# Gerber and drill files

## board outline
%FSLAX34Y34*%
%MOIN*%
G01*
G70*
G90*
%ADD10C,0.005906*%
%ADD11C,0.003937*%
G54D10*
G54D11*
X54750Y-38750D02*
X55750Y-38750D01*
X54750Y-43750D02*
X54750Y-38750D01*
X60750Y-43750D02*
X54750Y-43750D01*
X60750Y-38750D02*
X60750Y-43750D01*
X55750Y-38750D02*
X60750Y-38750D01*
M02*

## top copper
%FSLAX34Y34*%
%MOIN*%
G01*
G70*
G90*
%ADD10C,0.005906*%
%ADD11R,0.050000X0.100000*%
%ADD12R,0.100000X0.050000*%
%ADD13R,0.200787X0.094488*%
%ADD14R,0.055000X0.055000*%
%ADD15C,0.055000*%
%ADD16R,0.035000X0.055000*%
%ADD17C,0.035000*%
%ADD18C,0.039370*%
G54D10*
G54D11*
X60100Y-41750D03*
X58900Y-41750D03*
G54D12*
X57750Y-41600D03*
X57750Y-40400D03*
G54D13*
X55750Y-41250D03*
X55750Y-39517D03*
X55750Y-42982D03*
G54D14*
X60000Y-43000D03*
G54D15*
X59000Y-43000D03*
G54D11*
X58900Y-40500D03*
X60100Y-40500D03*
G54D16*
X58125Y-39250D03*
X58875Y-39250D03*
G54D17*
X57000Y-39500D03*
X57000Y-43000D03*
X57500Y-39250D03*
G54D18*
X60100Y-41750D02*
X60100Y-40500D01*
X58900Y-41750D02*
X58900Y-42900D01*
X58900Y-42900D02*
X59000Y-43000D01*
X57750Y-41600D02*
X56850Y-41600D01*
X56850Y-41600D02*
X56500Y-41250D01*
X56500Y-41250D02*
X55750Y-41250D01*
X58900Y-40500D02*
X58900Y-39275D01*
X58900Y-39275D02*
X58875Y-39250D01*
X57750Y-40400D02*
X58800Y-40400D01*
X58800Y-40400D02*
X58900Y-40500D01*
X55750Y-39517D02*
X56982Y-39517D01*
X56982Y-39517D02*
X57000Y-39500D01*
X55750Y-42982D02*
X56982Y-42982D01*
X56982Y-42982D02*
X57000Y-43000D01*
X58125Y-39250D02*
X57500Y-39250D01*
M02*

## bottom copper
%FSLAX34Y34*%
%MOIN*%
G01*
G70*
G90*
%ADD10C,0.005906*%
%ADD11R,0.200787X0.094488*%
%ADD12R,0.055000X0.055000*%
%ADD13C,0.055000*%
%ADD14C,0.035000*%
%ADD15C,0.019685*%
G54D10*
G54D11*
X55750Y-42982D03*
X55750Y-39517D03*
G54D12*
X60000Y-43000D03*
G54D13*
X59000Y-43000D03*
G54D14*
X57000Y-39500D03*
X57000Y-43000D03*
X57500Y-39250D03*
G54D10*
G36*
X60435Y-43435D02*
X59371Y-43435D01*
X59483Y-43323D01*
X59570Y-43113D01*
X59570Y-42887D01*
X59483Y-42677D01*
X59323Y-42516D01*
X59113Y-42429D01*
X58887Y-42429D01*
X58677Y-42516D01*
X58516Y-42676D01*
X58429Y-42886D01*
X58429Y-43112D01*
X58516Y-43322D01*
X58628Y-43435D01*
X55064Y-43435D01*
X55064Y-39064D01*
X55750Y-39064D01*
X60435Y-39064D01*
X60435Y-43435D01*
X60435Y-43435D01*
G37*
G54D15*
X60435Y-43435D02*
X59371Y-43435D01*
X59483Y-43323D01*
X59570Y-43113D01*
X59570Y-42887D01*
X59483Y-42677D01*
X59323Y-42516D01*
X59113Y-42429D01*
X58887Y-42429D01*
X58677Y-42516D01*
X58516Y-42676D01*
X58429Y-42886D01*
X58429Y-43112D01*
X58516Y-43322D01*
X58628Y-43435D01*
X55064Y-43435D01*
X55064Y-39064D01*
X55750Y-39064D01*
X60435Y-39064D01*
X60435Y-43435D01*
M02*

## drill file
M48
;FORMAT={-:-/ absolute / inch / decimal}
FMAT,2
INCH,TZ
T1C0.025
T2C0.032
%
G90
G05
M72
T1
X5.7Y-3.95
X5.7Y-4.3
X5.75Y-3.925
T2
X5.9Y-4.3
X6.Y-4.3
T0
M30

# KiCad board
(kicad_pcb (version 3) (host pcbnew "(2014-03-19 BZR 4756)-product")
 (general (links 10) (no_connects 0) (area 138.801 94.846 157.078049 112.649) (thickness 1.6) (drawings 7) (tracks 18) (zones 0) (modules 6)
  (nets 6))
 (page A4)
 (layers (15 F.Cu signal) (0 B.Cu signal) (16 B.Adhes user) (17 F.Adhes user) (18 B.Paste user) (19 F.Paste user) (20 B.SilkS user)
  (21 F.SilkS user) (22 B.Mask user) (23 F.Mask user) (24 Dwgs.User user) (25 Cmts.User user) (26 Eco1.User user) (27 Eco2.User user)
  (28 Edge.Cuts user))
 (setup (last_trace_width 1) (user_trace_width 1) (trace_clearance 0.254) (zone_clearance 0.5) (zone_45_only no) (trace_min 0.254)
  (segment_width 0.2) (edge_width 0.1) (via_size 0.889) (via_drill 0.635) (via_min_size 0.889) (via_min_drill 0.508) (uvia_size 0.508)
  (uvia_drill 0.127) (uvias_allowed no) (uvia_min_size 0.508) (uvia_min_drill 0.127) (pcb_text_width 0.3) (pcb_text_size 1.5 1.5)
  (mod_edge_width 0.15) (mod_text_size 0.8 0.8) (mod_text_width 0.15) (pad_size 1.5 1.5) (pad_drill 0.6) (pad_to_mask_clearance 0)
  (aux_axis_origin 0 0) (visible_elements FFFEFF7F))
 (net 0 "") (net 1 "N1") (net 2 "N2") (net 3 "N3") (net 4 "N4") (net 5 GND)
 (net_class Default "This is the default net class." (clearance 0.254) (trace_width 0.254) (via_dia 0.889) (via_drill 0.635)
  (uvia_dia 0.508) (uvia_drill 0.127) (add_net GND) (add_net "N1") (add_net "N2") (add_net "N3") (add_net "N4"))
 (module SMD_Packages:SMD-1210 (layer F.Cu) (at 151.13 106.045 180)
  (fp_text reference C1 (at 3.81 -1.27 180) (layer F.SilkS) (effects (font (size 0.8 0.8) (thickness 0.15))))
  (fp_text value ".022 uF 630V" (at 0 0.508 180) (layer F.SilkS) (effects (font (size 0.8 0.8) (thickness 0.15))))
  (pad 1 smd rect (at -1.524 0 180) (size 1.27 2.54) (layers F.Cu F.Paste F.Mask) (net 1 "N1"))
  (pad 2 smd rect (at 1.524 0 180) (size 1.27 2.54) (layers F.Cu F.Paste F.Mask) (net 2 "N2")))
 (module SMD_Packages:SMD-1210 (layer F.Cu) (at 146.685 104.14 90)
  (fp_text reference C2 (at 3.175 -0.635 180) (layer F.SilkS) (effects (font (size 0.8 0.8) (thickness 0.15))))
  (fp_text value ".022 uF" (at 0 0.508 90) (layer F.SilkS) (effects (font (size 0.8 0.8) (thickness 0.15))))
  (pad 1 smd rect (at -1.524 0 90) (size 1.27 2.54) (layers F.Cu F.Paste F.Mask) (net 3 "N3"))
  (pad 2 smd rect (at 1.524 0 90) (size 1.27 2.54) (layers F.Cu F.Paste F.Mask) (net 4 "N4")))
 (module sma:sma (layer F.Cu) (at 141.605 104.775)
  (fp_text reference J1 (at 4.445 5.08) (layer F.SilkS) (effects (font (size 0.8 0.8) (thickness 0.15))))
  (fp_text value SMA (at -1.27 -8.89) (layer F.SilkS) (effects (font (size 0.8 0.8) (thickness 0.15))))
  (pad 1 smd rect (at 0 0) (size 5.1 2.4) (layers F.Cu F.Paste F.Mask) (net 3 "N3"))
  (pad 2 smd rect (at 0 -4.4) (size 5.1 2.4) (layers F.Cu F.Paste F.Mask) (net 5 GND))
  (pad 3 smd rect (at 0 4.4) (size 5.1 2.4) (layers F.Cu F.Paste F.Mask) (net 5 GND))
  (pad 4 smd rect (at 0 4.4) (size 5.1 2.4) (layers B.Cu B.Paste B.Mask) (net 5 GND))
  (pad 5 smd rect (at 0 -4.4) (size 5.1 2.4) (layers B.Cu B.Paste B.Mask) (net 5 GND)))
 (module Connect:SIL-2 (layer F.Cu) (at 151.13 109.22 180)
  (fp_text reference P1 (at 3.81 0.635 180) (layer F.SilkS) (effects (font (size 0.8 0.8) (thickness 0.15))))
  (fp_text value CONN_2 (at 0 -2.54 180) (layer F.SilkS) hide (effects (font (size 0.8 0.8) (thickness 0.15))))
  (pad 1 thru_hole rect (at -1.27 0 180) (size 1.397 1.397) (drill 0.8128) (layers *.Cu *.Mask F.SilkS) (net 5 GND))
  (pad 2 thru_hole circle (at 1.27 0 180) (size 1.397 1.397) (drill 0.8128) (layers *.Cu *.Mask F.SilkS) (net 2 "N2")))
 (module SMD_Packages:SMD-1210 (layer F.Cu) (at 151.13 102.87)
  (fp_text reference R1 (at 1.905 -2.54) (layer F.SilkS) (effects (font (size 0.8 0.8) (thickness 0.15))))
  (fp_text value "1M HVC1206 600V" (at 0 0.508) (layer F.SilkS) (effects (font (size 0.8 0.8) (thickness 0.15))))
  (pad 1 smd rect (at -1.524 0) (size 1.27 2.54) (layers F.Cu F.Paste F.Mask) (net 4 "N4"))
  (pad 2 smd rect (at 1.524 0) (size 1.27 2.54) (layers F.Cu F.Paste F.Mask) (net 1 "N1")))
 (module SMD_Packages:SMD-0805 (layer F.Cu) (at 148.59 99.695)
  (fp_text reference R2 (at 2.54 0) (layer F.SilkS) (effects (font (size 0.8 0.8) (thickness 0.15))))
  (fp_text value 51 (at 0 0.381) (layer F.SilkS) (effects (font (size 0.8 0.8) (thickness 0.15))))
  (pad 1 smd rect (at -0.9525 0) (size 0.889 1.397) (layers F.Cu F.Paste F.Mask) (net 5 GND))
  (pad 2 smd rect (at 0.9525 0) (size 0.889 1.397) (layers F.Cu F.Paste F.Mask) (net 4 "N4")))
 (gr_line (start 139.065 98.425) (end 141.605 98.425) (angle 90) (layer Edge.Cuts) (width 0.1))
 (gr_line (start 139.065 111.125) (end 139.065 98.425) (angle 90) (layer Edge.Cuts) (width 0.1))
 (gr_line (start 154.305 111.125) (end 139.065 111.125) (angle 90) (layer Edge.Cuts) (width 0.1))
 (gr_line (start 154.305 98.425) (end 154.305 111.125) (angle 90) (layer Edge.Cuts) (width 0.1))
 (gr_line (start 141.605 98.425) (end 154.305 98.425) (angle 90) (layer Edge.Cuts) (width 0.1))
 (segment (start 152.654 106.045) (end 152.654 102.87) (width 1) (layer F.Cu) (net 1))
 (segment (start 149.606 106.045) (end 149.606 108.966) (width 1) (layer F.Cu) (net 2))
 (segment (start 149.606 108.966) (end 149.86 109.22) (width 1) (layer F.Cu) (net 2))
 (segment (start 146.685 105.664) (end 144.399 105.664) (width 1) (layer F.Cu) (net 3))
 (segment (start 144.399 105.664) (end 143.51 104.775) (width 1) (layer F.Cu) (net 3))
 (segment (start 143.51 104.775) (end 141.605 104.775) (width 1) (layer F.Cu) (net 3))
 (segment (start 149.606 102.87) (end 149.606 99.7585) (width 1) (layer F.Cu) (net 4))
 (segment (start 149.606 99.7585) (end 149.5425 99.695) (width 1) (layer F.Cu) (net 4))
 (segment (start 146.685 102.616) (end 149.352 102.616) (width 1) (layer F.Cu) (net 4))
 (segment (start 149.352 102.616) (end 149.606 102.87) (width 1) (layer F.Cu) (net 4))
 (segment (start 141.605 100.375) (end 144.735 100.375) (width 1) (layer F.Cu) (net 5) (status 400000))
 (via (at 144.78 100.33) (size 0.889) (layers F.Cu B.Cu) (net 5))
 (segment (start 144.735 100.375) (end 144.78 100.33) (width 1) (layer F.Cu) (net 5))
 (segment (start 141.605 109.175) (end 144.735 109.175) (width 1) (layer F.Cu) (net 5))
 (via (at 144.78 109.22) (size 0.889) (layers F.Cu B.Cu) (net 5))
 (segment (start 144.735 109.175) (end 144.78 109.22) (width 1) (layer F.Cu) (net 5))
 (segment (start 147.6375 99.695) (end 146.05 99.695) (width 1) (layer F.Cu) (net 5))
 (via (at 146.05 99.695) (size 0.889) (layers F.Cu B.Cu) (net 5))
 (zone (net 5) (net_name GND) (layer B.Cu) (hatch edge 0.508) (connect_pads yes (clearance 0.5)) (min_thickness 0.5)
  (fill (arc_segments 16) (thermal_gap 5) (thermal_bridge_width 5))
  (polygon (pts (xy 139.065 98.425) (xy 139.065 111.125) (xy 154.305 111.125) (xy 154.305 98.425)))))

